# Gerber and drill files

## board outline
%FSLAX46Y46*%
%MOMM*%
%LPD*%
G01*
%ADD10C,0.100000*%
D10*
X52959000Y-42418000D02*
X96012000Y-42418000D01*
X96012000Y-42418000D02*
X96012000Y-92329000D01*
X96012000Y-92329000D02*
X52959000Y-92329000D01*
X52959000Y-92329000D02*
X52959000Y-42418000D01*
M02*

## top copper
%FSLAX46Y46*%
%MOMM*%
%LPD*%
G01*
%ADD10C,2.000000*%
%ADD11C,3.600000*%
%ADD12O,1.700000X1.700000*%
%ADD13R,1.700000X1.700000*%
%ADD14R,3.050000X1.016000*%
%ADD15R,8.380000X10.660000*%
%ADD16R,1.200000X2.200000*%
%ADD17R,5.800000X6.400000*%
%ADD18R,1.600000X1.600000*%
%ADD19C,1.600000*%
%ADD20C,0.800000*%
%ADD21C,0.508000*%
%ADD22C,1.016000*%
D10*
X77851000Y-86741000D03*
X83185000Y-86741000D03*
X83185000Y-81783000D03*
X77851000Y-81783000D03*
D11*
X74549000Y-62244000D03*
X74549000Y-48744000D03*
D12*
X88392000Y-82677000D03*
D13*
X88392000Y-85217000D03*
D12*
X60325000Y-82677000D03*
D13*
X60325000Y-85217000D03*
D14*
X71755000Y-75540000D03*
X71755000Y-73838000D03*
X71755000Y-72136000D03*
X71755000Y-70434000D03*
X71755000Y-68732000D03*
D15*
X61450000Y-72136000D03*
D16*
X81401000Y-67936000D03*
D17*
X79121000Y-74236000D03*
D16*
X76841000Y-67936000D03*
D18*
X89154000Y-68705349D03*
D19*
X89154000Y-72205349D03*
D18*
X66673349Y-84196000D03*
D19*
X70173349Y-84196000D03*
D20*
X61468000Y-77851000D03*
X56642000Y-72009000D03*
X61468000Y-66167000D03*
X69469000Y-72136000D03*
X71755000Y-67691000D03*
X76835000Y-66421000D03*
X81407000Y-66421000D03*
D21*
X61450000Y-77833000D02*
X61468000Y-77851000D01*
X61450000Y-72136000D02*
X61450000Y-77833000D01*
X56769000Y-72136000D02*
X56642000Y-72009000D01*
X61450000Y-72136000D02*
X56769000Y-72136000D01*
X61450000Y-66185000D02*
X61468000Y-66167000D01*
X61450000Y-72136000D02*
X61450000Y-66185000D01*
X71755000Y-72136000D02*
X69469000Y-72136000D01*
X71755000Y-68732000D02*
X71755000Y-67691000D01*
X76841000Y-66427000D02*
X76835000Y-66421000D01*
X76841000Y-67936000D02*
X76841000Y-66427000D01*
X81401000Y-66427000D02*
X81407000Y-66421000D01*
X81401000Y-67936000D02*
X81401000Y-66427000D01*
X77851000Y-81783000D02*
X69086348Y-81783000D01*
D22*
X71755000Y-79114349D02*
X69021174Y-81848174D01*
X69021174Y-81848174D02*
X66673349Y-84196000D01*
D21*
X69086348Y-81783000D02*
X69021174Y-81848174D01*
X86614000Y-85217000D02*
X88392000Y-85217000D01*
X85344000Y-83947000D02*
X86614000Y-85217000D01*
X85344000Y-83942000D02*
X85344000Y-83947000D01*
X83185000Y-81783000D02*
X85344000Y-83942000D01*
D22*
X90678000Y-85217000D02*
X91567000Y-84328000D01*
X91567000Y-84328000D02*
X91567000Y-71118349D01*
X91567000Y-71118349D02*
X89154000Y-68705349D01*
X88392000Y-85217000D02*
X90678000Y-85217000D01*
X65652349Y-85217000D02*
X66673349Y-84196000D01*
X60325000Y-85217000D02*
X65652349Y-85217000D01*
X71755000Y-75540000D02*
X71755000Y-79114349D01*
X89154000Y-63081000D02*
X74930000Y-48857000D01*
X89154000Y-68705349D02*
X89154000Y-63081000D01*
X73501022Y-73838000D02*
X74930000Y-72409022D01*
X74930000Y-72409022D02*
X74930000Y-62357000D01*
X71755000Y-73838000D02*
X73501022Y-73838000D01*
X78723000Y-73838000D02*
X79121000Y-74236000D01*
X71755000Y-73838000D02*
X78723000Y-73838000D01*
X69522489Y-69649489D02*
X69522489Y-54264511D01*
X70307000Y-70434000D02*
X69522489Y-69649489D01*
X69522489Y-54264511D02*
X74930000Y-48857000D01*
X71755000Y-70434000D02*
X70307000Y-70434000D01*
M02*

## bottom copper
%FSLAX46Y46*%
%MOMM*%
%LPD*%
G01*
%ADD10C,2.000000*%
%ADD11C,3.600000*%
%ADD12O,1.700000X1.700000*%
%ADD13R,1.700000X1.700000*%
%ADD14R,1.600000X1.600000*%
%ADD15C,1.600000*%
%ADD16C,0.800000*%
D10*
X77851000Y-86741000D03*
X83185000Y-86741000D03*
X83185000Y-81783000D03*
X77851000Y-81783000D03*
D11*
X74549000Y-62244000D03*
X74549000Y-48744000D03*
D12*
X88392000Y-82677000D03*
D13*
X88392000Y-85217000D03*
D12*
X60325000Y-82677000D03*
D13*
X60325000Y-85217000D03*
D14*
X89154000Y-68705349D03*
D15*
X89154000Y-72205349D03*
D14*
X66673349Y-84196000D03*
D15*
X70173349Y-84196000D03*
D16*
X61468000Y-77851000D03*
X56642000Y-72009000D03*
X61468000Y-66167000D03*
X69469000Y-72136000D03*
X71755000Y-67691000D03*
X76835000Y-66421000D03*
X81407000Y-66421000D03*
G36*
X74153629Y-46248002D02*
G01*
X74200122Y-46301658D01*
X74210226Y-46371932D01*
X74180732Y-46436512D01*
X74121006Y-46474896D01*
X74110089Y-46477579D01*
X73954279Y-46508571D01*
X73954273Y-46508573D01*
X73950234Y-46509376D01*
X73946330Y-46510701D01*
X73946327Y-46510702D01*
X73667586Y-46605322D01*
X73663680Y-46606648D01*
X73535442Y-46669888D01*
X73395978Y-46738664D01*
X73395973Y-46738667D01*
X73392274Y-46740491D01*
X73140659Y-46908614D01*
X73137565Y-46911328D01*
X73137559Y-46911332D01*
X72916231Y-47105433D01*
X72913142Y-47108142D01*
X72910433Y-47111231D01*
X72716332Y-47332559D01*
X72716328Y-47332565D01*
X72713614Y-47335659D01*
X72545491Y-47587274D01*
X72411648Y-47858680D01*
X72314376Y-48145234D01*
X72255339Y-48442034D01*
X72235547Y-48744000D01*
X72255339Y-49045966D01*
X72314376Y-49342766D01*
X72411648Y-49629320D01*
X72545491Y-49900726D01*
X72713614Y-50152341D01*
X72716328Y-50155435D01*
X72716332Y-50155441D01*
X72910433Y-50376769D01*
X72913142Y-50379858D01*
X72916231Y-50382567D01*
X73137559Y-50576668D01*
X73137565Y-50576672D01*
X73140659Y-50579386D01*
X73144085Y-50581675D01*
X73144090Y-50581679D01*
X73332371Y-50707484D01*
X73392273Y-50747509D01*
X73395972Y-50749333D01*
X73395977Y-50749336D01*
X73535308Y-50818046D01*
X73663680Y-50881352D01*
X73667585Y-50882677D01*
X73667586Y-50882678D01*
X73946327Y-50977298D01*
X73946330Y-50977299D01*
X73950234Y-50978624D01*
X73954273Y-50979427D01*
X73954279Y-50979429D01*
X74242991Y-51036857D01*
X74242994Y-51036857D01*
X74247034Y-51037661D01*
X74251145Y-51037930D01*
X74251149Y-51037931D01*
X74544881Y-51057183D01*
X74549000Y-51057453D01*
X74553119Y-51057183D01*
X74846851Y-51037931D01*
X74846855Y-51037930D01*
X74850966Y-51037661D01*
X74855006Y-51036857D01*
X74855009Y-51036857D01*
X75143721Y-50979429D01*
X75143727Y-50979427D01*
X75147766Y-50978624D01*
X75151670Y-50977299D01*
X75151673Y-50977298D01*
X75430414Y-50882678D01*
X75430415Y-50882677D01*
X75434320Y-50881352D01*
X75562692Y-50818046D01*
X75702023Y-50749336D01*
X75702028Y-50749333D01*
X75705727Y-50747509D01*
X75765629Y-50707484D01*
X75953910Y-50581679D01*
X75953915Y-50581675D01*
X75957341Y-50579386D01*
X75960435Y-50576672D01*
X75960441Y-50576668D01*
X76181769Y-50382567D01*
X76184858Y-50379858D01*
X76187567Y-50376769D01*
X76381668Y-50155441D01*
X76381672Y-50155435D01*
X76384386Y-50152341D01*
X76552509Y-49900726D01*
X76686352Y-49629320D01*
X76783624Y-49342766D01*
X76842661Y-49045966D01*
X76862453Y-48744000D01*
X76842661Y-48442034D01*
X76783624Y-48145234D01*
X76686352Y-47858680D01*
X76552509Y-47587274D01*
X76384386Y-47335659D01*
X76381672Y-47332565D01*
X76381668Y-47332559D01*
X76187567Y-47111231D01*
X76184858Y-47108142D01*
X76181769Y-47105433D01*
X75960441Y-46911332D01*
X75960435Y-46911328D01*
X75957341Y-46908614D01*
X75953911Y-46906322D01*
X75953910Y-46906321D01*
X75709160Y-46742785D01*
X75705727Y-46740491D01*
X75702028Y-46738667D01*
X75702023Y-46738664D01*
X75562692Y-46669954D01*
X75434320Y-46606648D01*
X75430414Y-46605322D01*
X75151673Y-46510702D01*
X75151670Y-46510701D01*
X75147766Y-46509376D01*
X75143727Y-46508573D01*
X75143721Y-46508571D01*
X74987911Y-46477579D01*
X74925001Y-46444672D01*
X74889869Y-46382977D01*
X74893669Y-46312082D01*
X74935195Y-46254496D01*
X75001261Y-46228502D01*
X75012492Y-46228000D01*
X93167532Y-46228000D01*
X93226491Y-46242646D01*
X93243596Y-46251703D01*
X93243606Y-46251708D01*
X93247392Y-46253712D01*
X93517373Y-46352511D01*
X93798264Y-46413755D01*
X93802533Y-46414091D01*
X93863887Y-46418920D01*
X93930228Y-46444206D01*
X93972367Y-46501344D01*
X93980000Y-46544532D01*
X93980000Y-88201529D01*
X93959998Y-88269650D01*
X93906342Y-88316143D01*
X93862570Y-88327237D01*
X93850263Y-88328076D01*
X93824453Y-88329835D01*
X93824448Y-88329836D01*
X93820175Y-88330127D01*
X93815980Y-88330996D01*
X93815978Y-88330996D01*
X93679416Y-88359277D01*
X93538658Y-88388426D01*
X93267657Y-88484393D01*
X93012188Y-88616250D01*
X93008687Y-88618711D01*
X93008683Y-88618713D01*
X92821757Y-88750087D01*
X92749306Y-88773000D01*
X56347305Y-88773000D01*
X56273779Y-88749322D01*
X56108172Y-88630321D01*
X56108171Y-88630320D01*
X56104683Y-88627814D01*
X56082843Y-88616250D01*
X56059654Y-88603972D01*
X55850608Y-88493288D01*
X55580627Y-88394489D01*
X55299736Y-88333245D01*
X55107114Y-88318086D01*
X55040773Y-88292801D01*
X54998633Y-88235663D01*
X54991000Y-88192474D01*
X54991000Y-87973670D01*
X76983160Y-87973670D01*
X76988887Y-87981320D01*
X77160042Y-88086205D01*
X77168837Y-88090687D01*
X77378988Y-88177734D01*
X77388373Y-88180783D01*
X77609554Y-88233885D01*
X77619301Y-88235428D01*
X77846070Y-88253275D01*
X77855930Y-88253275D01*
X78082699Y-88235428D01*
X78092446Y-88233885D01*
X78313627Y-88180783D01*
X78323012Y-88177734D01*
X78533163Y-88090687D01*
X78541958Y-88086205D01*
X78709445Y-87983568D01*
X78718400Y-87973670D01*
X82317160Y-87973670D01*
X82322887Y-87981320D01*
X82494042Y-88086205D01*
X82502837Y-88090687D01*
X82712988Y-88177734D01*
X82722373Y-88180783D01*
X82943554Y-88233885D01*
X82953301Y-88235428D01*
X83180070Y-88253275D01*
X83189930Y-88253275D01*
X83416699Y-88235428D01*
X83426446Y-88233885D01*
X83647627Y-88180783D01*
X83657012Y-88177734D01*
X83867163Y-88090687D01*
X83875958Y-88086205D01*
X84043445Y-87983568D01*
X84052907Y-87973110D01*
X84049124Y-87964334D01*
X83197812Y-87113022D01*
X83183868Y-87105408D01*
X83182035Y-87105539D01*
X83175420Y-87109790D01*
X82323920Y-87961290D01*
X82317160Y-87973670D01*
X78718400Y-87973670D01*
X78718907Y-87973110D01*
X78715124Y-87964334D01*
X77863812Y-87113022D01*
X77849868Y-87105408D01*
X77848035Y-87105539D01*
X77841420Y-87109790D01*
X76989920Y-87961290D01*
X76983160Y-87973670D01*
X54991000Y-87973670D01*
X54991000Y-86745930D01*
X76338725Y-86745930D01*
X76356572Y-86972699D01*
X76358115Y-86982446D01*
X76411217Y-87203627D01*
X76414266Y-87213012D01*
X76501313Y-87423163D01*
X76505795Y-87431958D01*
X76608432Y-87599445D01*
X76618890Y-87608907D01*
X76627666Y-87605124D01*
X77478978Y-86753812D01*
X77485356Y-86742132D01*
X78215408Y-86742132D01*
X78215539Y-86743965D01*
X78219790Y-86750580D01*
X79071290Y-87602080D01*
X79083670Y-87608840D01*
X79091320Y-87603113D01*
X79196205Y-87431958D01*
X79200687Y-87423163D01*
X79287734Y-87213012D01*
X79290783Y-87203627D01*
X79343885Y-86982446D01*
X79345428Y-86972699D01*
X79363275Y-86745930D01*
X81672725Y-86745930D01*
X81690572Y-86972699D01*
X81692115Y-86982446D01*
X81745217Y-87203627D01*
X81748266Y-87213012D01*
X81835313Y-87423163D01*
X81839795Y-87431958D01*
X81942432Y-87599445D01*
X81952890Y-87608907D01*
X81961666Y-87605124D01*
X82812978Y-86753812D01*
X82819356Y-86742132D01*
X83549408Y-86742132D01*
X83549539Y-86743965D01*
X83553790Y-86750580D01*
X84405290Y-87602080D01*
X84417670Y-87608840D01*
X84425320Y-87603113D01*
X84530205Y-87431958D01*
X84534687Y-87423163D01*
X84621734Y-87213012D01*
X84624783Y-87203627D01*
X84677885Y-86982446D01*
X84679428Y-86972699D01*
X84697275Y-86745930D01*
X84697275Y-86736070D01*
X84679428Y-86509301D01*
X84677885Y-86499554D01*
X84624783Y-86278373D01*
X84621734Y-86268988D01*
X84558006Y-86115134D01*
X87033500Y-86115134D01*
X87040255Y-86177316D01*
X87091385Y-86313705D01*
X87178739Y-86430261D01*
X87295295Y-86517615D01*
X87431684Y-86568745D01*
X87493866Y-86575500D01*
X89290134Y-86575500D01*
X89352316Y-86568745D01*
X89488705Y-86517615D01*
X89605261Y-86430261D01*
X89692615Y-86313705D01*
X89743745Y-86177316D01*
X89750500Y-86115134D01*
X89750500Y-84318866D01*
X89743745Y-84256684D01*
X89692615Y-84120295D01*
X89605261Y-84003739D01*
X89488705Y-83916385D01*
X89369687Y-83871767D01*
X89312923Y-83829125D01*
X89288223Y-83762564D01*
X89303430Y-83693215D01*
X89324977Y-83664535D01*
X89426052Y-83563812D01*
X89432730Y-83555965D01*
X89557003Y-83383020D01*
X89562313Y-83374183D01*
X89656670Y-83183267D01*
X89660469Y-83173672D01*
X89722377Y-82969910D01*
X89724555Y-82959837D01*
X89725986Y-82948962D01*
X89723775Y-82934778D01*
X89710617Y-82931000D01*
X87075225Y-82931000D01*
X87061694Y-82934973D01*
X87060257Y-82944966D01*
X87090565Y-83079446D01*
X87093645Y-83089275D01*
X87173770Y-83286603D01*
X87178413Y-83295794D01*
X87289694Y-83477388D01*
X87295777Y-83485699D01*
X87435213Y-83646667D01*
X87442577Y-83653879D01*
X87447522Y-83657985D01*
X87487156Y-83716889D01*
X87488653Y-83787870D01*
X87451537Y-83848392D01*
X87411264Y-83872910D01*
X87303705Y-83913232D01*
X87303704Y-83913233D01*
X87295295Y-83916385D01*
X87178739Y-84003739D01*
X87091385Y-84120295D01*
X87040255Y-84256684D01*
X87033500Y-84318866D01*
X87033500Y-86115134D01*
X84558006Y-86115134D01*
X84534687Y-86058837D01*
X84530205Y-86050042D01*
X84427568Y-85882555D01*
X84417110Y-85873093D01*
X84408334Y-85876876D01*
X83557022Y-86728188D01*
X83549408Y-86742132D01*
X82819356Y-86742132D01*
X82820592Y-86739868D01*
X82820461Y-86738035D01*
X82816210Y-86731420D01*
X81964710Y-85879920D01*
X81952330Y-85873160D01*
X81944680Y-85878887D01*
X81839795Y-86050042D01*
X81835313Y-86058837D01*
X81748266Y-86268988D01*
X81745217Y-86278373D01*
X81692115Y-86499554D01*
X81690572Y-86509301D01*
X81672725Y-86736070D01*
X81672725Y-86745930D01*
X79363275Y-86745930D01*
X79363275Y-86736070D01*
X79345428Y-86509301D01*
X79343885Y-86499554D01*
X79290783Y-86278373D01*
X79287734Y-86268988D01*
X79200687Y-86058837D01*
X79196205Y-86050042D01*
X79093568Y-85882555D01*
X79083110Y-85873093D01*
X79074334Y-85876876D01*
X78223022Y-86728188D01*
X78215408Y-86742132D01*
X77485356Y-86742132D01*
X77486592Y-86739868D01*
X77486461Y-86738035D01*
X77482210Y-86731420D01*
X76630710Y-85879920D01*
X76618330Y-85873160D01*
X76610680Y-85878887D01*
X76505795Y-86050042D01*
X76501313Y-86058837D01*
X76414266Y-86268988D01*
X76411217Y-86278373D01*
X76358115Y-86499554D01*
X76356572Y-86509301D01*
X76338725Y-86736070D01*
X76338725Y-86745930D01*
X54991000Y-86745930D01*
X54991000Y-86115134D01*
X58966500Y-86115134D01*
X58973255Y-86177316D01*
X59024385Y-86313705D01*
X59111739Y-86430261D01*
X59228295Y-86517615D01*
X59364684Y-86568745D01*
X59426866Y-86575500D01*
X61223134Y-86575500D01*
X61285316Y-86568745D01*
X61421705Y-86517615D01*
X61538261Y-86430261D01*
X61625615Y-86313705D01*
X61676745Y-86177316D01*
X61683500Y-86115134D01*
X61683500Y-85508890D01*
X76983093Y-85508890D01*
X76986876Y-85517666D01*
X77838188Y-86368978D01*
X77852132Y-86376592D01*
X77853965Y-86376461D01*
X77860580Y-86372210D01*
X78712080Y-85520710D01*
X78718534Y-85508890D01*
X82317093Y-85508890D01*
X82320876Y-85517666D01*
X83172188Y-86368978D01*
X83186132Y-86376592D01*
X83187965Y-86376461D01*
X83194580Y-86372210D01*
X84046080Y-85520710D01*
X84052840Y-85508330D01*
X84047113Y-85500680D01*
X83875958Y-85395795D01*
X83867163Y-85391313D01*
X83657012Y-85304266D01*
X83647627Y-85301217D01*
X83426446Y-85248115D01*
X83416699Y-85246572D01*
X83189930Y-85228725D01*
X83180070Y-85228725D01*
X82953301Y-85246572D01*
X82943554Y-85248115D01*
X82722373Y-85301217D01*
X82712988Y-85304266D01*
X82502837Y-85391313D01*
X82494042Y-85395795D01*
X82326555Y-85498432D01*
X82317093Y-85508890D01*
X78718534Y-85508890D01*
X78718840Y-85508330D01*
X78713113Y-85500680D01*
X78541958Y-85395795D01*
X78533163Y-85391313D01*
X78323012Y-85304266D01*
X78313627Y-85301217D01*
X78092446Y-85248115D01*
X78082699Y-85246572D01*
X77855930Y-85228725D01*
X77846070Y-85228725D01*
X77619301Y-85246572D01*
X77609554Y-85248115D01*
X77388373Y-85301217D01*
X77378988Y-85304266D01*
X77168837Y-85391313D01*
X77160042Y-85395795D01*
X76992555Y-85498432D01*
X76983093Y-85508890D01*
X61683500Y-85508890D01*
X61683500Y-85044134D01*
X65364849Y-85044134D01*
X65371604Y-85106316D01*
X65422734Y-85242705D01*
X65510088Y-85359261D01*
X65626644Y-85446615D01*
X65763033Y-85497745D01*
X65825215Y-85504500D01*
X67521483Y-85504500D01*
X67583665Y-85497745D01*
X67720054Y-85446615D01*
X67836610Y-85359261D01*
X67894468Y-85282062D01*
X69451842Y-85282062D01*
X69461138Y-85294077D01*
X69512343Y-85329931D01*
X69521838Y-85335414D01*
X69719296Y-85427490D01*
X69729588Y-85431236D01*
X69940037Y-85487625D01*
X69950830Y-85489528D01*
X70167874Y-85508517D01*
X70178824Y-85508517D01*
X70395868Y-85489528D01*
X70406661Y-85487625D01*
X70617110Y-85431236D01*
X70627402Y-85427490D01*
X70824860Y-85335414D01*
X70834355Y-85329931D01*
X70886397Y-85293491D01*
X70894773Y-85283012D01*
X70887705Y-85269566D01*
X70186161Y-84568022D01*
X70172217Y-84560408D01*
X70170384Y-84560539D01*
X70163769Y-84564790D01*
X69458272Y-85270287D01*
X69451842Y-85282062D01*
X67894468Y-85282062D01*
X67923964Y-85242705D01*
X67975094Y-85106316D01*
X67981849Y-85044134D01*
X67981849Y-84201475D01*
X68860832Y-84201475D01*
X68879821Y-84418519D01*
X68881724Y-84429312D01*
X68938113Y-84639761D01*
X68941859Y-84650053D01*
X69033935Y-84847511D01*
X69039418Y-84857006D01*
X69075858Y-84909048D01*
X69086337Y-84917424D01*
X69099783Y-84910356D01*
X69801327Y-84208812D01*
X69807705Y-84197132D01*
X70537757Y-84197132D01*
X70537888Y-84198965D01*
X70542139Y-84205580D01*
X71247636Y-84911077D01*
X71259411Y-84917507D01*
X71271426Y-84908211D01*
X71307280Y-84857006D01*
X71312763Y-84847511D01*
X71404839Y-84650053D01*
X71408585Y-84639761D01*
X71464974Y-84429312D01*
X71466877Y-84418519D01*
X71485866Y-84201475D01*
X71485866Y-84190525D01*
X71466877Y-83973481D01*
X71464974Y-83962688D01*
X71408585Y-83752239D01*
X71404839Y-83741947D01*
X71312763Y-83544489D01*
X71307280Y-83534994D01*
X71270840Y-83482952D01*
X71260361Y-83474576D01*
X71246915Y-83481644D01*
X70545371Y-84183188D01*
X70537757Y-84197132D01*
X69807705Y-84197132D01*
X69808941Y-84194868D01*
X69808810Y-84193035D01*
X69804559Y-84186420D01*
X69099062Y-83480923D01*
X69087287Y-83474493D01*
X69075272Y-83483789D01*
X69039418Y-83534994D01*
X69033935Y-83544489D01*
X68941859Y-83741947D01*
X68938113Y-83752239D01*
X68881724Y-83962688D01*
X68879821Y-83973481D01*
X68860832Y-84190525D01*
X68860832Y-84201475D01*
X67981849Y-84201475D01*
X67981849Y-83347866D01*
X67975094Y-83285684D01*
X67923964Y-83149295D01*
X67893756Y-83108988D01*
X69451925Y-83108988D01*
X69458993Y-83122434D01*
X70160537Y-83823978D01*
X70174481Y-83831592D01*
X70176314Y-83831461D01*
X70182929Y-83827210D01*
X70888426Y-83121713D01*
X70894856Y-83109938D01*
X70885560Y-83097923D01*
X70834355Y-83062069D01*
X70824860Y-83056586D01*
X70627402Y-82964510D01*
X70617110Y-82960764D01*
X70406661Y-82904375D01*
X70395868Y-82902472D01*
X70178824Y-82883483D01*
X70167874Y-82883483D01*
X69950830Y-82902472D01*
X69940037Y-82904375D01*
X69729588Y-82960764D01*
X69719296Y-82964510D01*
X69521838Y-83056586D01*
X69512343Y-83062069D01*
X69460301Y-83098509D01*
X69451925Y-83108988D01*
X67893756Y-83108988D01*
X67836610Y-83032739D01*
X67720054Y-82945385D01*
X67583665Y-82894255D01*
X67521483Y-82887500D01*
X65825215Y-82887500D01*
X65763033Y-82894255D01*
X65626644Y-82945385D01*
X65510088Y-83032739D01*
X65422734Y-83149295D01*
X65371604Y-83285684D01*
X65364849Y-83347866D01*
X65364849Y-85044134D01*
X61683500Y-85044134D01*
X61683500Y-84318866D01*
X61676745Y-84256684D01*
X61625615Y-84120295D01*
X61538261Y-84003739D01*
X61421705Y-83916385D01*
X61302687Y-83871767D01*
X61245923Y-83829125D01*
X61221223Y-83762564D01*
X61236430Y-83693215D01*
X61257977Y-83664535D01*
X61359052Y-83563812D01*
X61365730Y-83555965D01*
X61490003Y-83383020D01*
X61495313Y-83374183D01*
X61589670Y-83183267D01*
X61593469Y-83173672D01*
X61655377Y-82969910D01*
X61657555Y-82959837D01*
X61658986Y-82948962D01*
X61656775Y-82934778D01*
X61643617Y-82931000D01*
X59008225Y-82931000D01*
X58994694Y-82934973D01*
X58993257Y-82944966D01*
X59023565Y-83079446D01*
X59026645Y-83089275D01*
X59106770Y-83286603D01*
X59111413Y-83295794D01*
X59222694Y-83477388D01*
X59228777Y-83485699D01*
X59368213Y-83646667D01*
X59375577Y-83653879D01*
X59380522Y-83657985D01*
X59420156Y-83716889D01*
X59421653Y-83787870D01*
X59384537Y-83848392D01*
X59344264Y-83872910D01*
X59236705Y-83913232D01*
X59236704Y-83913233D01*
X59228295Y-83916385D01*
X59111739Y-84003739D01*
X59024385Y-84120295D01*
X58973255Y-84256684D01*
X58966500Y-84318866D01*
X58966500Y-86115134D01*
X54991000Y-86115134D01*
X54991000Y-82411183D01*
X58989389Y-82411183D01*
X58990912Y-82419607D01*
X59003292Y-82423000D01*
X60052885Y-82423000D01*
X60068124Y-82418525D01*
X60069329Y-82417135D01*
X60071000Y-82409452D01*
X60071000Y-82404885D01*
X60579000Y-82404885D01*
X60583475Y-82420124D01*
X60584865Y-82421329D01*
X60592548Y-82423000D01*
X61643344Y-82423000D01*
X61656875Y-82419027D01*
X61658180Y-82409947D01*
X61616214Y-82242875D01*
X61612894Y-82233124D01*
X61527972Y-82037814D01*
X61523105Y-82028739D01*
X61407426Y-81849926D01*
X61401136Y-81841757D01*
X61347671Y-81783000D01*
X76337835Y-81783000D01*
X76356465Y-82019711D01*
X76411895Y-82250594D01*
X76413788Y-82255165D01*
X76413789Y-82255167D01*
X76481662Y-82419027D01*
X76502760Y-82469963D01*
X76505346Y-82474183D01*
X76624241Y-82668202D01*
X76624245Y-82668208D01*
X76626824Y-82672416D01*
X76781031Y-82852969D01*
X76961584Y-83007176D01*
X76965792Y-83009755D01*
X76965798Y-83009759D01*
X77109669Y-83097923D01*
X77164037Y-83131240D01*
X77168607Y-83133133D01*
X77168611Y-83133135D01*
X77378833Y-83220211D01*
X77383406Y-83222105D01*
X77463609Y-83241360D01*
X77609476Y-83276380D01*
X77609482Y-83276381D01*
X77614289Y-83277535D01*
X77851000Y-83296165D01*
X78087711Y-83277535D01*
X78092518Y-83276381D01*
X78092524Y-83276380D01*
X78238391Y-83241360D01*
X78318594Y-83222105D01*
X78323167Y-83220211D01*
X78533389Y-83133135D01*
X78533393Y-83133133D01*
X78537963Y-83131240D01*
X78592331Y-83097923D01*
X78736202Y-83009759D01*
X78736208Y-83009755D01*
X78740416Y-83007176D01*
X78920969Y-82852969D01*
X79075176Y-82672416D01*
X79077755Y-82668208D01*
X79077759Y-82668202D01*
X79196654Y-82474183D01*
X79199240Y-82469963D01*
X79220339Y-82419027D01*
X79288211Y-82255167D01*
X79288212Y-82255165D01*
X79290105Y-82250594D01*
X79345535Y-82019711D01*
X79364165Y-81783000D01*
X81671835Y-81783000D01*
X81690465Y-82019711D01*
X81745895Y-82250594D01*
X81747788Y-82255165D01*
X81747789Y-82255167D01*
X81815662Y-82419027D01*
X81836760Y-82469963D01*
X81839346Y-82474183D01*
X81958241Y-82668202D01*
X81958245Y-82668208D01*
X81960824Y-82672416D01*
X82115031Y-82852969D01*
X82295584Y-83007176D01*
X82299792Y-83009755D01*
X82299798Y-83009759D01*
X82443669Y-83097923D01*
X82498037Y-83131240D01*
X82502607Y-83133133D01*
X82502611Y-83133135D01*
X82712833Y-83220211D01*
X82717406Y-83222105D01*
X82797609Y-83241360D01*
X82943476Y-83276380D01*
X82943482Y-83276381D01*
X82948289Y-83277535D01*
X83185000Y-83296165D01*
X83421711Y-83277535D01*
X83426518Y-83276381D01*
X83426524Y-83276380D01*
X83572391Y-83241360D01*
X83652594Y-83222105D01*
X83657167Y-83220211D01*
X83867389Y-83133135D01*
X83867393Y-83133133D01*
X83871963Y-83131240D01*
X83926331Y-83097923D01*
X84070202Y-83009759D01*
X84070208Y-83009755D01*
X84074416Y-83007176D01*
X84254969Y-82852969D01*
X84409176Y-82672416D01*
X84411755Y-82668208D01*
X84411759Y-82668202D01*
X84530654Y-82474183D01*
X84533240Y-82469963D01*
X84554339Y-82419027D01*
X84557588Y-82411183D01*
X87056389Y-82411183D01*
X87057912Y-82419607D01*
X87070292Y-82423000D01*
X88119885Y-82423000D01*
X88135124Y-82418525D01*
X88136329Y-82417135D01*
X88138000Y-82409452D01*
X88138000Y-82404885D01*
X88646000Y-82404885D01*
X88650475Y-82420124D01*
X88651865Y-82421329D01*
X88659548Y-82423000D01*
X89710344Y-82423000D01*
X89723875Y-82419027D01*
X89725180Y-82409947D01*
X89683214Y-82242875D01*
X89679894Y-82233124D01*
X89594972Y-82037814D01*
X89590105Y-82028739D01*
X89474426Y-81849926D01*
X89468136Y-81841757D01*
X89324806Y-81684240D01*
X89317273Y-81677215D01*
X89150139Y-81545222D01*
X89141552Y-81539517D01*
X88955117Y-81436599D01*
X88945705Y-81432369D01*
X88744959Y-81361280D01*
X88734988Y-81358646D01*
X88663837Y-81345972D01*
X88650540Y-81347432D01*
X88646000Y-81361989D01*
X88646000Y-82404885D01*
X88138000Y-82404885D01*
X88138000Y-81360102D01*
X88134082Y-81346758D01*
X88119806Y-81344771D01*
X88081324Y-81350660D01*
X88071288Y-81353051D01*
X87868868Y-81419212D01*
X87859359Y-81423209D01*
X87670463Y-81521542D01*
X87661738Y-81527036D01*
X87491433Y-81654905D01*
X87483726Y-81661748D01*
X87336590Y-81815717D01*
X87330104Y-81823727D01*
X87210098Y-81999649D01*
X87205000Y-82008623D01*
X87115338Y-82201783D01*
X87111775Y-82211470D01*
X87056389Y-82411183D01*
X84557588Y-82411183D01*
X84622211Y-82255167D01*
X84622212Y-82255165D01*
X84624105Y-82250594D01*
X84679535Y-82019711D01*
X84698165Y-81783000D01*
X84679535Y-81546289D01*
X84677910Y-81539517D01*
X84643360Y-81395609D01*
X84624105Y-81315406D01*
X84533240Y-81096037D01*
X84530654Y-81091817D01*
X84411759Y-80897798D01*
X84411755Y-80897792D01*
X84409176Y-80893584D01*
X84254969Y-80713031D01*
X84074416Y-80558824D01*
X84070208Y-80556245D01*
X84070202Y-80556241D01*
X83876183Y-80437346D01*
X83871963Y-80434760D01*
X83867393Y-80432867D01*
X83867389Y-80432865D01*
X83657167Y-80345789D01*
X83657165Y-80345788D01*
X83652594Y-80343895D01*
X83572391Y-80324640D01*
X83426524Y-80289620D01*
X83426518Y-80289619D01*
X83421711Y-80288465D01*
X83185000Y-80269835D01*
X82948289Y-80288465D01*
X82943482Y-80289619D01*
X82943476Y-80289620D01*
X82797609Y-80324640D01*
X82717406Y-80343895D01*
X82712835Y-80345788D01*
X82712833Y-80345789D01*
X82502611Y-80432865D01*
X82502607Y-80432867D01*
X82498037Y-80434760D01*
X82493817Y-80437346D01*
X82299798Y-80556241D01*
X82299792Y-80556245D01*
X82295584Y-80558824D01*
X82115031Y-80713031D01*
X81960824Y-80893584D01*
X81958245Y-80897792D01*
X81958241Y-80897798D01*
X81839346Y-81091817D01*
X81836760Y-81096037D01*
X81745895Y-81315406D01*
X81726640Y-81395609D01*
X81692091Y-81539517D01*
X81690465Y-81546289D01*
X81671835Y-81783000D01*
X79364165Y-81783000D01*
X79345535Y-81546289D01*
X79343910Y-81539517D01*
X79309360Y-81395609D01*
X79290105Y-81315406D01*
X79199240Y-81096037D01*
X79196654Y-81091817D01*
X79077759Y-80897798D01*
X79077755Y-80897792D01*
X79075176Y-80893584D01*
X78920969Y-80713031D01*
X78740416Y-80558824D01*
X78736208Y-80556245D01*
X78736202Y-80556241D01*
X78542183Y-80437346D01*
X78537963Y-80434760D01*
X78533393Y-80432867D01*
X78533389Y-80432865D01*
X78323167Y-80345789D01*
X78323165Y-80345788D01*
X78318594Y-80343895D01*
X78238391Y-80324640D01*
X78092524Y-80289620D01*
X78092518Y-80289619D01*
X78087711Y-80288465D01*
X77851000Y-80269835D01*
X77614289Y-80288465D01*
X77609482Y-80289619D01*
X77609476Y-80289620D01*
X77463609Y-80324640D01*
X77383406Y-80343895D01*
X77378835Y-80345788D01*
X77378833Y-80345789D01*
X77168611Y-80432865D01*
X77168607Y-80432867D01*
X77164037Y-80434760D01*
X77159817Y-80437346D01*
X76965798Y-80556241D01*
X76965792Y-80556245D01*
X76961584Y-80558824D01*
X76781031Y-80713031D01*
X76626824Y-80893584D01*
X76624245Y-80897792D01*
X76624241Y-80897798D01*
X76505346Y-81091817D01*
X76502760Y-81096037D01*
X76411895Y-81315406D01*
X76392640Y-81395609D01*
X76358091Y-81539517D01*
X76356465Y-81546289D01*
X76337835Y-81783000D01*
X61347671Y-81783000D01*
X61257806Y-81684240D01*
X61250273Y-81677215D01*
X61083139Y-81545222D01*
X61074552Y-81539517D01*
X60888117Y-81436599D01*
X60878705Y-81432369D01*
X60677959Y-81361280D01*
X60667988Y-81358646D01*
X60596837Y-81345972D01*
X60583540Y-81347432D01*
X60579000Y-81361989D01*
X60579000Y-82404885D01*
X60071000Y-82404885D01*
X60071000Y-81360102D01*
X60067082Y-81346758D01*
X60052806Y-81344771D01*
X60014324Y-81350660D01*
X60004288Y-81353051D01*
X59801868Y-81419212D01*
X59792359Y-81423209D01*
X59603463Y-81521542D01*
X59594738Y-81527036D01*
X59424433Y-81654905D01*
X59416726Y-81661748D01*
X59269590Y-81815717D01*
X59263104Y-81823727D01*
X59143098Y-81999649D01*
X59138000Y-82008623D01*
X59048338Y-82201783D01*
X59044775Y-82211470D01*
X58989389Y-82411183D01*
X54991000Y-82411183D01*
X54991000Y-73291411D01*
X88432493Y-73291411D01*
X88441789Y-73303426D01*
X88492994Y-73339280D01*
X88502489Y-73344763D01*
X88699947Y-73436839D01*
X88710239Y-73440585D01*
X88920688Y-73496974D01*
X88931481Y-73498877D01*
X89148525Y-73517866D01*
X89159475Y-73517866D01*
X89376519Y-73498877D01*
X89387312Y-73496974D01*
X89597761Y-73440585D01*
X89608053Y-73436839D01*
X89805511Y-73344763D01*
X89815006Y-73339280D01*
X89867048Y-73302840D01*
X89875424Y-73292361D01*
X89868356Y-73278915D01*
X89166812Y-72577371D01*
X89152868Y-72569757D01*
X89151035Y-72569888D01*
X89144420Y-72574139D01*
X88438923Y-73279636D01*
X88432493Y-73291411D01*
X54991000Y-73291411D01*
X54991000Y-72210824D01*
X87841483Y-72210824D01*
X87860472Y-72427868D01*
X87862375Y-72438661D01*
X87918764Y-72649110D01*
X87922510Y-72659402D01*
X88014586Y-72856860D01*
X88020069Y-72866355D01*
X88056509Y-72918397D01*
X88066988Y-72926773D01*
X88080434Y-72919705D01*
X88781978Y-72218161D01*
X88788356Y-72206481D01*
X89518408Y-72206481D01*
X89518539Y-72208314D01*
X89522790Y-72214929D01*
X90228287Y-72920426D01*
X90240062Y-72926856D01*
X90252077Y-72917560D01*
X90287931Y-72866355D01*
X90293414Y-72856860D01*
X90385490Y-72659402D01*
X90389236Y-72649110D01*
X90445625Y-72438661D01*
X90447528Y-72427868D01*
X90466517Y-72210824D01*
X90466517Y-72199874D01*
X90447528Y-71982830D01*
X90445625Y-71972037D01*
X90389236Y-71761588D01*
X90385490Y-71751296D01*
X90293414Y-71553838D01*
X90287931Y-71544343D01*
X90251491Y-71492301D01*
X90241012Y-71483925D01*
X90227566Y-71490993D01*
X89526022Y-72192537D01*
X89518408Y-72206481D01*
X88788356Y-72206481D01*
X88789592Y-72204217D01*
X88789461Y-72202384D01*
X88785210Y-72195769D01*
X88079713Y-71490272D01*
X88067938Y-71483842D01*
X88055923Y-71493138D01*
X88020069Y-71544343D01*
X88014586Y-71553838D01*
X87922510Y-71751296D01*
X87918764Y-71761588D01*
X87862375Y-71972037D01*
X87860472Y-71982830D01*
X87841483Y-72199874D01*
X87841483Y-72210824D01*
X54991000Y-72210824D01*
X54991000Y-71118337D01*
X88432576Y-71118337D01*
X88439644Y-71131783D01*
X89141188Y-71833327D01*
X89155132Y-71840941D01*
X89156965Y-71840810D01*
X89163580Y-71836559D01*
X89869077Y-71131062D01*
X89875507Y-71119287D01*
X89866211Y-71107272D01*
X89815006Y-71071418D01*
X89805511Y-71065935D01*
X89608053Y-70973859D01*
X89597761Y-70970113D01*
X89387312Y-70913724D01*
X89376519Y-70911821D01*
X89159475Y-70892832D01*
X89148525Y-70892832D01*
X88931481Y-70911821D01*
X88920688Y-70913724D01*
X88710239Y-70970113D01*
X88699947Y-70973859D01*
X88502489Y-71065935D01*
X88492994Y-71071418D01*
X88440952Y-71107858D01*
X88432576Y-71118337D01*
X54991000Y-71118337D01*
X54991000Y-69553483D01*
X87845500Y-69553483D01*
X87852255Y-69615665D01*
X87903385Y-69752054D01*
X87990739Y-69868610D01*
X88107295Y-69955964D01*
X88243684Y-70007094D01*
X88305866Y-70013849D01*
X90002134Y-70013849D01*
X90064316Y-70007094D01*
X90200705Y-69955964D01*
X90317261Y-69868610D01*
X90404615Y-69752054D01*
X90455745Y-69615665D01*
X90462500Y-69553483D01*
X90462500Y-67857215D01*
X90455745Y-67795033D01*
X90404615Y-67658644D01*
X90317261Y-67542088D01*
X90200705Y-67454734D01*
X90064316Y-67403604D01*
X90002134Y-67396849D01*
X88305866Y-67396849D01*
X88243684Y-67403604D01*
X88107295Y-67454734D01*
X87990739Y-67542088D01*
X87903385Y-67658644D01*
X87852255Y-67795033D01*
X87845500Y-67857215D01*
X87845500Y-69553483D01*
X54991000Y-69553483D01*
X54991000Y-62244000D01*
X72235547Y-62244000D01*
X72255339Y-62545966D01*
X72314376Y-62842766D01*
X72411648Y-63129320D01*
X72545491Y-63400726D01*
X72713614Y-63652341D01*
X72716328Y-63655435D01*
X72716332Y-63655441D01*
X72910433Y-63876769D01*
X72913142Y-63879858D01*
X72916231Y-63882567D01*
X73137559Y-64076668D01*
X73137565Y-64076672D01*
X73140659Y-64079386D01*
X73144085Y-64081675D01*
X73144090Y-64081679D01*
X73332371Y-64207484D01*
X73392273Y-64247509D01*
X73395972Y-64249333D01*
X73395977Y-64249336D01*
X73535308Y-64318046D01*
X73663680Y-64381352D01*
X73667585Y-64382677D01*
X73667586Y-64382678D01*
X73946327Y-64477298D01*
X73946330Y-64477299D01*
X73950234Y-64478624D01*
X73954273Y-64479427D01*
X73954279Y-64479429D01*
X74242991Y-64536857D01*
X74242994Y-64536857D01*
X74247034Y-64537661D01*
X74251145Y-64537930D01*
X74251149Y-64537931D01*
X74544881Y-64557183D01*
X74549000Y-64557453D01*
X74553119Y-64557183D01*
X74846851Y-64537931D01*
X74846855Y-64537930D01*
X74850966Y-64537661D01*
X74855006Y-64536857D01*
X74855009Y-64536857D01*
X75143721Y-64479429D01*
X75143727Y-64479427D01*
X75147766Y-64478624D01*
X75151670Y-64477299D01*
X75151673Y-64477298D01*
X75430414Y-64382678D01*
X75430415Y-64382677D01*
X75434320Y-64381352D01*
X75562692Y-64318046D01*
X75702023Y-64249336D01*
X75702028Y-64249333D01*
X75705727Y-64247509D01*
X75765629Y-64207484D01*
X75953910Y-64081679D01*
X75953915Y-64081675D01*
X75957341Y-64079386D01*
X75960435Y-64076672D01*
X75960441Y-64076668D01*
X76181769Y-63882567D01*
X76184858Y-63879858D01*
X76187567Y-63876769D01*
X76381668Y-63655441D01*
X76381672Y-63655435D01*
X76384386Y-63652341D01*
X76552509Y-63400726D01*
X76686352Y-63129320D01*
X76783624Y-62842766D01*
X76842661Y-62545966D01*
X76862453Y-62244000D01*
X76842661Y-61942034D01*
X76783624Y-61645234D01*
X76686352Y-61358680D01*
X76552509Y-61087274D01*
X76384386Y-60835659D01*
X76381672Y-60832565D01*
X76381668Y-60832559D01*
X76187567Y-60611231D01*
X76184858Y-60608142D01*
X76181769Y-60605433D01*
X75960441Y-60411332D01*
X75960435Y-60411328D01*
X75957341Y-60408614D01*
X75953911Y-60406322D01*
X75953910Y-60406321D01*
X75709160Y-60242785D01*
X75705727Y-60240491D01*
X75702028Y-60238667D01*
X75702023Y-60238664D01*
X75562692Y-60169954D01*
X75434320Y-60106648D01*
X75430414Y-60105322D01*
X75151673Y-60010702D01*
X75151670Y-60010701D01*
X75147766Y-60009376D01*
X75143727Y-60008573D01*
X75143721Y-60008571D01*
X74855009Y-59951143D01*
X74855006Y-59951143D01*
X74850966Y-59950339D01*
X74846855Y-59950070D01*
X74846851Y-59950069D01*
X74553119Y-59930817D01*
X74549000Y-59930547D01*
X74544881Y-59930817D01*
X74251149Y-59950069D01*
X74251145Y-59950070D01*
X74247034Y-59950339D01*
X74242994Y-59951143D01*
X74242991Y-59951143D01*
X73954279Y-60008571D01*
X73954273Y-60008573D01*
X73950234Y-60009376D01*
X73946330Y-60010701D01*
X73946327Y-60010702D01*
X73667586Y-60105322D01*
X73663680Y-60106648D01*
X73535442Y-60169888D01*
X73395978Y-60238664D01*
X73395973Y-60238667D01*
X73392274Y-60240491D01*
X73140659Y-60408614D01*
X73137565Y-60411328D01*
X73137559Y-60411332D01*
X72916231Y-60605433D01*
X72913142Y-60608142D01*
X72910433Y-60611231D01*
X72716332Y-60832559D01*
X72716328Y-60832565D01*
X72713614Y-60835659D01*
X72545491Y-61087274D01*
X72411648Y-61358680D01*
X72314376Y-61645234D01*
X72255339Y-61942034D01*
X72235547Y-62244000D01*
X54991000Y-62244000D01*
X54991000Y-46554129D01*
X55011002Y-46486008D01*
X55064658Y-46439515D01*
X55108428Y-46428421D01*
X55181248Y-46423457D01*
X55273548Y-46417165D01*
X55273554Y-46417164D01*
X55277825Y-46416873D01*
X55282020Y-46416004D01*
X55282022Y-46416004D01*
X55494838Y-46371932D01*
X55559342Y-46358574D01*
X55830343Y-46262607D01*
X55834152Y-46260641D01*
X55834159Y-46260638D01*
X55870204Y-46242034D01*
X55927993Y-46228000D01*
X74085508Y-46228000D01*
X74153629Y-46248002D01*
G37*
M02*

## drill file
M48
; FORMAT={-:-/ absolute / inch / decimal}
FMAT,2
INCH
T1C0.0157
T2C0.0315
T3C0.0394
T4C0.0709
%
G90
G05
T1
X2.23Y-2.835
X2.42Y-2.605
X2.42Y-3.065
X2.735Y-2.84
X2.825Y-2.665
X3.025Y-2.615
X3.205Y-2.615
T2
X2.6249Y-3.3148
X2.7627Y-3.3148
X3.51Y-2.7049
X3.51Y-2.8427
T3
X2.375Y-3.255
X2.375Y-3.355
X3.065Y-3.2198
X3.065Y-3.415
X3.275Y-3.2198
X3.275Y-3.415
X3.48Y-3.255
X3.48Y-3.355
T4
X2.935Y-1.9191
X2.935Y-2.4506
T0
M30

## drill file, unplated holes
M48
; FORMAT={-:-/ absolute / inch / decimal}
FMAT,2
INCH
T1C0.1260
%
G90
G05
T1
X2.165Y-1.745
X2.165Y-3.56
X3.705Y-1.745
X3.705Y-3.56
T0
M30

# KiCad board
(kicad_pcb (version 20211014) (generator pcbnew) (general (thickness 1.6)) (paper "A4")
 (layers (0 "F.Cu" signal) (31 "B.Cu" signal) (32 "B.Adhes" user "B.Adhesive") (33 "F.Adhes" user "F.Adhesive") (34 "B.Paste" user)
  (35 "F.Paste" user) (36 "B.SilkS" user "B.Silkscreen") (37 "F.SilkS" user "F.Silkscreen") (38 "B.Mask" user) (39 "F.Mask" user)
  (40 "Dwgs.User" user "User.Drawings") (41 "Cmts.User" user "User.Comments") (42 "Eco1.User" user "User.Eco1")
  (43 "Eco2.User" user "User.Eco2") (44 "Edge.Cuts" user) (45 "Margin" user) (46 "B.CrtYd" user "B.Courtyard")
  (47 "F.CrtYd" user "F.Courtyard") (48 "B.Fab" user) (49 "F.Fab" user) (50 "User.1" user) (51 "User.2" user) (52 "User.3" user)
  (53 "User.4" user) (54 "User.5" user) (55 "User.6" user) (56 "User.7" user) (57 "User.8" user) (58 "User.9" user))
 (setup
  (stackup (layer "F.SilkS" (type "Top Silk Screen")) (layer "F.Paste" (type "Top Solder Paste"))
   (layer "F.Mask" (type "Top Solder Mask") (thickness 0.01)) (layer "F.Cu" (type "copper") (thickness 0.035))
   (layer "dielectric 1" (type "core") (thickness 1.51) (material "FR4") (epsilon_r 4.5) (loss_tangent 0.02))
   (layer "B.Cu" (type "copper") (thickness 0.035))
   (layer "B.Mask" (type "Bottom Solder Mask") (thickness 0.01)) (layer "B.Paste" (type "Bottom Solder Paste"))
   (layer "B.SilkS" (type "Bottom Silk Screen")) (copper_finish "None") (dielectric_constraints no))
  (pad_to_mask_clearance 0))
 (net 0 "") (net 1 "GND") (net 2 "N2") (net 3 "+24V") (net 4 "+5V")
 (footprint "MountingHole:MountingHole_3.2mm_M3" (layer "F.Cu") (at 94.107 90.424)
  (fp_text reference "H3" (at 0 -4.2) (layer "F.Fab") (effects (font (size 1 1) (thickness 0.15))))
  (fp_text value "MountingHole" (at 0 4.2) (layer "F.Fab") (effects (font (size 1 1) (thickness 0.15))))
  (pad "" np_thru_hole circle (at 0 0) (size 3.2 3.2) (drill 3.2) (layers *.Cu *.Mask)))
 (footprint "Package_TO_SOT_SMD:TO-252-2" (layer "F.Cu") (at 79.121 72.136 -90)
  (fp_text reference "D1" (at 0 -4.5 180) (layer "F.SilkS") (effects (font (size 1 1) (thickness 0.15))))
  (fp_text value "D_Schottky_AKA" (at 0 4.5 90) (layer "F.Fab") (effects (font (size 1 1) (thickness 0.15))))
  (pad "" smd rect (at 3.775 -1.525 270) (size 3.05 2.75) (layers "F.Paste"))
  (pad "" smd rect (at 0.425 1.525 270) (size 3.05 2.75) (layers "F.Paste"))
  (pad "" smd rect (at 3.775 1.525 270) (size 3.05 2.75) (layers "F.Paste"))
  (pad "" smd rect (at 0.425 -1.525 270) (size 3.05 2.75) (layers "F.Paste"))
  (pad "1" smd rect (at -4.2 -2.28 270) (size 2.2 1.2) (layers "F.Cu" "F.Paste" "F.Mask") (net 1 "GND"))
  (pad "2" smd rect (at 2.1 0 270) (size 6.4 5.8) (layers "F.Cu" "F.Mask") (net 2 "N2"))
  (pad "3" smd rect (at -4.2 2.28 270) (size 2.2 1.2) (layers "F.Cu" "F.Paste" "F.Mask") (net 1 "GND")))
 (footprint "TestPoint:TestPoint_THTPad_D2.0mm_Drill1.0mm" (layer "F.Cu") (at 77.851 81.783)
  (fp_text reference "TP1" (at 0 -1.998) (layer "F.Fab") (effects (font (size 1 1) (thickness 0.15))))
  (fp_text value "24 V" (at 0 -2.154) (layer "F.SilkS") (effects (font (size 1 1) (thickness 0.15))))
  (pad "1" thru_hole circle (at 0 0) (size 2 2) (drill 1) (layers *.Cu *.Mask) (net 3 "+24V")))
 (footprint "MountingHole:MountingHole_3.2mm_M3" (layer "F.Cu") (at 54.991 90.424)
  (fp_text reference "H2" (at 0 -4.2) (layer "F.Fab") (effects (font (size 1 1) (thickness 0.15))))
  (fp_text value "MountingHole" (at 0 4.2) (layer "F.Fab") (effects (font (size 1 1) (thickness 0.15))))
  (pad "" np_thru_hole circle (at 0 0) (size 3.2 3.2) (drill 3.2) (layers *.Cu *.Mask)))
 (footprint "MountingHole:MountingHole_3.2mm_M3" (layer "F.Cu") (at 54.991 44.323)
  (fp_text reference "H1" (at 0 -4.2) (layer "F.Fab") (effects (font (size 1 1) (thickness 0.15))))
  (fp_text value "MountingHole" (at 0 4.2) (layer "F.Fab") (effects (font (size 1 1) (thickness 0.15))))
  (pad "" np_thru_hole circle (at 0 0) (size 3.2 3.2) (drill 3.2) (layers *.Cu *.Mask)))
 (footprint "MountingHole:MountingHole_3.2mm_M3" (layer "F.Cu") (at 94.107 44.323)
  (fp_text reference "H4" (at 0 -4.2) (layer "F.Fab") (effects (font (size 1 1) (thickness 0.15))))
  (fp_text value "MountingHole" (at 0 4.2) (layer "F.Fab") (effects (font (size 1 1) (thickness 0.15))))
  (pad "" np_thru_hole circle (at 0 0) (size 3.2 3.2) (drill 3.2) (layers *.Cu *.Mask)))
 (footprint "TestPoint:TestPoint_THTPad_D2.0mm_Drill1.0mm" (layer "F.Cu") (at 77.851 86.741)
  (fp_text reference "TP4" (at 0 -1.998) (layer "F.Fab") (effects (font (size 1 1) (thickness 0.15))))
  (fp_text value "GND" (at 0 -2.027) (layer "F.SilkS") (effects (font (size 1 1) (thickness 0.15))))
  (pad "1" thru_hole circle (at 0 0) (size 2 2) (drill 1) (layers *.Cu *.Mask) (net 1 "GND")))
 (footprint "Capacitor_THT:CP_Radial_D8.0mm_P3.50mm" (layer "F.Cu") (at 66.673349 84.196)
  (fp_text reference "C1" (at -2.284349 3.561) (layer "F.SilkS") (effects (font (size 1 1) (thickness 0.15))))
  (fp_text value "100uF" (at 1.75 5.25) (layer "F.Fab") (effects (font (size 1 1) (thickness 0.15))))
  (pad "1" thru_hole rect (at 0 0) (size 1.6 1.6) (drill 0.8) (layers *.Cu *.Mask) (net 3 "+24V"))
  (pad "2" thru_hole circle (at 3.5 0) (size 1.6 1.6) (drill 0.8) (layers *.Cu *.Mask) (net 1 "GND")))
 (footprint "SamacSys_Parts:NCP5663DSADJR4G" (layer "F.Cu") (at 59.055 72.136)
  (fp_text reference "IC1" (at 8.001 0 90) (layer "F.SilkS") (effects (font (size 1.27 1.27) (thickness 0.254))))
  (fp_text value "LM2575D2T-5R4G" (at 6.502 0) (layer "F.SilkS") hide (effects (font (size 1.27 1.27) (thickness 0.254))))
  (pad "1" smd rect locked (at 12.7 3.404 90) (size 1.016 3.05) (layers "F.Cu" "F.Paste" "F.Mask") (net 3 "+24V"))
  (pad "2" smd rect locked (at 12.7 1.702 90) (size 1.016 3.05) (layers "F.Cu" "F.Paste" "F.Mask") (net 2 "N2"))
  (pad "3" smd rect locked (at 12.7 0 90) (size 1.016 3.05) (layers "F.Cu" "F.Paste" "F.Mask") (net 1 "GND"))
  (pad "4" smd rect locked (at 12.7 -1.702 90) (size 1.016 3.05) (layers "F.Cu" "F.Paste" "F.Mask") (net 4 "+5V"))
  (pad "5" smd rect locked (at 12.7 -3.404 90) (size 1.016 3.05) (layers "F.Cu" "F.Paste" "F.Mask") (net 1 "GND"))
  (pad "6" smd rect locked (at 2.395 0) (size 8.38 10.66) (layers "F.Cu" "F.Paste" "F.Mask") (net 1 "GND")))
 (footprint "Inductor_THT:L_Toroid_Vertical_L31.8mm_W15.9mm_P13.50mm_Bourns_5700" (layer "F.Cu") (at 74.549 62.244 180)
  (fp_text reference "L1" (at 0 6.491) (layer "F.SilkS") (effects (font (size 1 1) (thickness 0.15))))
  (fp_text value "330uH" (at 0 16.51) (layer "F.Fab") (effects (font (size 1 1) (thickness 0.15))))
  (pad "1" thru_hole circle (at 0 0 180) (size 3.6 3.6) (drill 1.8) (layers *.Cu *.Mask) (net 2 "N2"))
  (pad "2" thru_hole circle (at 0 13.5 180) (size 3.6 3.6) (drill 1.8) (layers *.Cu *.Mask) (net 4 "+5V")))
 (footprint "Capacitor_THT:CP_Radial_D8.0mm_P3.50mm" (layer "F.Cu") (at 89.154 68.705349 -90)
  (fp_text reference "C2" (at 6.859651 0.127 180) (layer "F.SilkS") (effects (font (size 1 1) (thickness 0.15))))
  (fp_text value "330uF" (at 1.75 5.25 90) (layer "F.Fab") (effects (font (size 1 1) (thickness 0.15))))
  (pad "1" thru_hole rect (at 0 0 270) (size 1.6 1.6) (drill 0.8) (layers *.Cu *.Mask) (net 4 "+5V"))
  (pad "2" thru_hole circle (at 3.5 0 270) (size 1.6 1.6) (drill 0.8) (layers *.Cu *.Mask) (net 1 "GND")))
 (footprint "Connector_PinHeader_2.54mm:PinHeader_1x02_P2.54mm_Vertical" (layer "F.Cu") (at 88.392 85.217 180)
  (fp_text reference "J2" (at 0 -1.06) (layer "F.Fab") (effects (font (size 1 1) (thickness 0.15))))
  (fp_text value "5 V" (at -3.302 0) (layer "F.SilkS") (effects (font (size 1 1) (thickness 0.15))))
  (pad "1" thru_hole rect (at 0 0 180) (size 1.7 1.7) (drill 1) (layers *.Cu *.Mask) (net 4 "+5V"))
  (pad "2" thru_hole oval (at 0 2.54 180) (size 1.7 1.7) (drill 1) (layers *.Cu *.Mask) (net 1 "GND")))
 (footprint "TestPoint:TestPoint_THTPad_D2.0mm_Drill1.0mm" (layer "F.Cu") (at 83.185 81.783)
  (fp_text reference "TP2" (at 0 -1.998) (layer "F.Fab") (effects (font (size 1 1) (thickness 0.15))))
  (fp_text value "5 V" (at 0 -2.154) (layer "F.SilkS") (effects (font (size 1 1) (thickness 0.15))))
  (pad "1" thru_hole circle (at 0 0) (size 2 2) (drill 1) (layers *.Cu *.Mask) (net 4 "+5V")))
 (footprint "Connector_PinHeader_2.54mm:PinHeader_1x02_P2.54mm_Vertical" (layer "F.Cu") (at 60.325 85.217 180)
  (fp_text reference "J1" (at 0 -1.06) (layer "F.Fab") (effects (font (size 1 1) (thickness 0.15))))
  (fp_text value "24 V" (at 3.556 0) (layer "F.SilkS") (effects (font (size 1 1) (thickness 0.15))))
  (pad "1" thru_hole rect (at 0 0 180) (size 1.7 1.7) (drill 1) (layers *.Cu *.Mask) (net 3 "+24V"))
  (pad "2" thru_hole oval (at 0 2.54 180) (size 1.7 1.7) (drill 1) (layers *.Cu *.Mask) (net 1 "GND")))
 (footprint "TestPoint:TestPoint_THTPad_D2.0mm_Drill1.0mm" (layer "F.Cu") (at 83.185 86.741)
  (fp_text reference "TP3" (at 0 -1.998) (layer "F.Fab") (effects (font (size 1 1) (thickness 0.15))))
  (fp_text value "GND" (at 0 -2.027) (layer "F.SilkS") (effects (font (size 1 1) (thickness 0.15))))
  (pad "1" thru_hole circle (at 0 0) (size 2 2) (drill 1) (layers *.Cu *.Mask) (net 1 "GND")))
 (gr_rect (start 52.959 42.418) (end 96.012 92.329) (layer "Edge.Cuts") (width 0.1) (fill none))
 (segment (start 77.851 81.783) (end 69.086348 81.783) (width 0.508) (layer "F.Cu") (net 3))
 (segment (start 71.755 79.114349) (end 69.021174 81.848174) (width 1.016) (layer "F.Cu") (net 3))
 (segment (start 65.652349 85.217) (end 66.673349 84.196) (width 1.016) (layer "F.Cu") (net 3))
 (segment (start 60.325 85.217) (end 65.652349 85.217) (width 1.016) (layer "F.Cu") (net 3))
 (segment (start 69.086348 81.783) (end 69.021174 81.848174) (width 0.508) (layer "F.Cu") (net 3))
 (segment (start 71.755 75.54) (end 71.755 79.114349) (width 1.016) (layer "F.Cu") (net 3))
 (segment (start 69.021174 81.848174) (end 66.673349 84.196) (width 1.016) (layer "F.Cu") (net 3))
 (segment (start 56.769 72.136) (end 56.642 72.009) (width 0.508) (layer "F.Cu") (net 1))
 (segment (start 61.45 72.136) (end 61.45 77.833) (width 0.508) (layer "F.Cu") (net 1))
 (segment (start 61.45 66.185) (end 61.468 66.167) (width 0.508) (layer "F.Cu") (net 1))
 (segment (start 61.45 77.833) (end 61.468 77.851) (width 0.508) (layer "F.Cu") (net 1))
 (segment (start 81.401 67.936) (end 81.401 66.427) (width 0.508) (layer "F.Cu") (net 1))
 (segment (start 76.841 66.427) (end 76.835 66.421) (width 0.508) (layer "F.Cu") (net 1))
 (segment (start 71.755 72.136) (end 69.469 72.136) (width 0.508) (layer "F.Cu") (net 1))
 (segment (start 76.841 67.936) (end 76.841 66.427) (width 0.508) (layer "F.Cu") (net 1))
 (segment (start 61.45 72.136) (end 56.769 72.136) (width 0.508) (layer "F.Cu") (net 1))
 (segment (start 71.755 68.732) (end 71.755 67.691) (width 0.508) (layer "F.Cu") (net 1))
 (segment (start 81.401 66.427) (end 81.407 66.421) (width 0.508) (layer "F.Cu") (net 1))
 (segment (start 61.45 72.136) (end 61.45 66.185) (width 0.508) (layer "F.Cu") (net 1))
 (via (at 61.468 66.167) (size 0.8) (drill 0.4) (layers "F.Cu" "B.Cu") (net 1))
 (via (at 81.407 66.421) (size 0.8) (drill 0.4) (layers "F.Cu" "B.Cu") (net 1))
 (via (at 71.755 67.691) (size 0.8) (drill 0.4) (layers "F.Cu" "B.Cu") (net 1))
 (via (at 76.835 66.421) (size 0.8) (drill 0.4) (layers "F.Cu" "B.Cu") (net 1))
 (via (at 61.468 77.851) (size 0.8) (drill 0.4) (layers "F.Cu" "B.Cu") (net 1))
 (via (at 56.642 72.009) (size 0.8) (drill 0.4) (layers "F.Cu" "B.Cu") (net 1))
 (via (at 69.469 72.136) (size 0.8) (drill 0.4) (layers "F.Cu" "B.Cu") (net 1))
 (segment (start 88.392 85.217) (end 90.678 85.217) (width 1.016) (layer "F.Cu") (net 4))
 (segment (start 89.154 63.081) (end 74.93 48.857) (width 1.016) (layer "F.Cu") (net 4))
 (segment (start 86.614 85.217) (end 88.392 85.217) (width 0.508) (layer "F.Cu") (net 4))
 (segment (start 69.522489 54.264511) (end 74.93 48.857) (width 1.016) (layer "F.Cu") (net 4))
 (segment (start 83.185 81.783) (end 85.344 83.942) (width 0.508) (layer "F.Cu") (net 4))
 (segment (start 70.307 70.434) (end 69.522489 69.649489) (width 1.016) (layer "F.Cu") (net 4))
 (segment (start 89.154 68.705349) (end 89.154 63.081) (width 1.016) (layer "F.Cu") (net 4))
 (segment (start 91.567 84.328) (end 91.567 71.118349) (width 1.016) (layer "F.Cu") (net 4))
 (segment (start 90.678 85.217) (end 91.567 84.328) (width 1.016) (layer "F.Cu") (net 4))
 (segment (start 85.344 83.942) (end 85.344 83.947) (width 0.508) (layer "F.Cu") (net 4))
 (segment (start 91.567 71.118349) (end 89.154 68.705349) (width 1.016) (layer "F.Cu") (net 4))
 (segment (start 71.755 70.434) (end 70.307 70.434) (width 1.016) (layer "F.Cu") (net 4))
 (segment (start 85.344 83.947) (end 86.614 85.217) (width 0.508) (layer "F.Cu") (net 4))
 (segment (start 69.522489 69.649489) (end 69.522489 54.264511) (width 1.016) (layer "F.Cu") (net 4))
 (segment (start 73.501022 73.838) (end 74.93 72.409022) (width 1.016) (layer "F.Cu") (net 2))
 (segment (start 74.93 72.409022) (end 74.93 62.357) (width 1.016) (layer "F.Cu") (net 2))
 (segment (start 78.723 73.838) (end 79.121 74.236) (width 1.016) (layer "F.Cu") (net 2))
 (segment (start 71.755 73.838) (end 78.723 73.838) (width 1.016) (layer "F.Cu") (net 2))
 (segment (start 71.755 73.838) (end 73.501022 73.838) (width 1.016) (layer "F.Cu") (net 2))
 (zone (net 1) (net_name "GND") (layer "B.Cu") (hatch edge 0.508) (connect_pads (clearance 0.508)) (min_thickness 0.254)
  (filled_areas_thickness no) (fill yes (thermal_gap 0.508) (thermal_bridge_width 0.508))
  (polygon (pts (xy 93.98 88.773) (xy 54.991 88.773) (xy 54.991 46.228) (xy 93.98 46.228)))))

